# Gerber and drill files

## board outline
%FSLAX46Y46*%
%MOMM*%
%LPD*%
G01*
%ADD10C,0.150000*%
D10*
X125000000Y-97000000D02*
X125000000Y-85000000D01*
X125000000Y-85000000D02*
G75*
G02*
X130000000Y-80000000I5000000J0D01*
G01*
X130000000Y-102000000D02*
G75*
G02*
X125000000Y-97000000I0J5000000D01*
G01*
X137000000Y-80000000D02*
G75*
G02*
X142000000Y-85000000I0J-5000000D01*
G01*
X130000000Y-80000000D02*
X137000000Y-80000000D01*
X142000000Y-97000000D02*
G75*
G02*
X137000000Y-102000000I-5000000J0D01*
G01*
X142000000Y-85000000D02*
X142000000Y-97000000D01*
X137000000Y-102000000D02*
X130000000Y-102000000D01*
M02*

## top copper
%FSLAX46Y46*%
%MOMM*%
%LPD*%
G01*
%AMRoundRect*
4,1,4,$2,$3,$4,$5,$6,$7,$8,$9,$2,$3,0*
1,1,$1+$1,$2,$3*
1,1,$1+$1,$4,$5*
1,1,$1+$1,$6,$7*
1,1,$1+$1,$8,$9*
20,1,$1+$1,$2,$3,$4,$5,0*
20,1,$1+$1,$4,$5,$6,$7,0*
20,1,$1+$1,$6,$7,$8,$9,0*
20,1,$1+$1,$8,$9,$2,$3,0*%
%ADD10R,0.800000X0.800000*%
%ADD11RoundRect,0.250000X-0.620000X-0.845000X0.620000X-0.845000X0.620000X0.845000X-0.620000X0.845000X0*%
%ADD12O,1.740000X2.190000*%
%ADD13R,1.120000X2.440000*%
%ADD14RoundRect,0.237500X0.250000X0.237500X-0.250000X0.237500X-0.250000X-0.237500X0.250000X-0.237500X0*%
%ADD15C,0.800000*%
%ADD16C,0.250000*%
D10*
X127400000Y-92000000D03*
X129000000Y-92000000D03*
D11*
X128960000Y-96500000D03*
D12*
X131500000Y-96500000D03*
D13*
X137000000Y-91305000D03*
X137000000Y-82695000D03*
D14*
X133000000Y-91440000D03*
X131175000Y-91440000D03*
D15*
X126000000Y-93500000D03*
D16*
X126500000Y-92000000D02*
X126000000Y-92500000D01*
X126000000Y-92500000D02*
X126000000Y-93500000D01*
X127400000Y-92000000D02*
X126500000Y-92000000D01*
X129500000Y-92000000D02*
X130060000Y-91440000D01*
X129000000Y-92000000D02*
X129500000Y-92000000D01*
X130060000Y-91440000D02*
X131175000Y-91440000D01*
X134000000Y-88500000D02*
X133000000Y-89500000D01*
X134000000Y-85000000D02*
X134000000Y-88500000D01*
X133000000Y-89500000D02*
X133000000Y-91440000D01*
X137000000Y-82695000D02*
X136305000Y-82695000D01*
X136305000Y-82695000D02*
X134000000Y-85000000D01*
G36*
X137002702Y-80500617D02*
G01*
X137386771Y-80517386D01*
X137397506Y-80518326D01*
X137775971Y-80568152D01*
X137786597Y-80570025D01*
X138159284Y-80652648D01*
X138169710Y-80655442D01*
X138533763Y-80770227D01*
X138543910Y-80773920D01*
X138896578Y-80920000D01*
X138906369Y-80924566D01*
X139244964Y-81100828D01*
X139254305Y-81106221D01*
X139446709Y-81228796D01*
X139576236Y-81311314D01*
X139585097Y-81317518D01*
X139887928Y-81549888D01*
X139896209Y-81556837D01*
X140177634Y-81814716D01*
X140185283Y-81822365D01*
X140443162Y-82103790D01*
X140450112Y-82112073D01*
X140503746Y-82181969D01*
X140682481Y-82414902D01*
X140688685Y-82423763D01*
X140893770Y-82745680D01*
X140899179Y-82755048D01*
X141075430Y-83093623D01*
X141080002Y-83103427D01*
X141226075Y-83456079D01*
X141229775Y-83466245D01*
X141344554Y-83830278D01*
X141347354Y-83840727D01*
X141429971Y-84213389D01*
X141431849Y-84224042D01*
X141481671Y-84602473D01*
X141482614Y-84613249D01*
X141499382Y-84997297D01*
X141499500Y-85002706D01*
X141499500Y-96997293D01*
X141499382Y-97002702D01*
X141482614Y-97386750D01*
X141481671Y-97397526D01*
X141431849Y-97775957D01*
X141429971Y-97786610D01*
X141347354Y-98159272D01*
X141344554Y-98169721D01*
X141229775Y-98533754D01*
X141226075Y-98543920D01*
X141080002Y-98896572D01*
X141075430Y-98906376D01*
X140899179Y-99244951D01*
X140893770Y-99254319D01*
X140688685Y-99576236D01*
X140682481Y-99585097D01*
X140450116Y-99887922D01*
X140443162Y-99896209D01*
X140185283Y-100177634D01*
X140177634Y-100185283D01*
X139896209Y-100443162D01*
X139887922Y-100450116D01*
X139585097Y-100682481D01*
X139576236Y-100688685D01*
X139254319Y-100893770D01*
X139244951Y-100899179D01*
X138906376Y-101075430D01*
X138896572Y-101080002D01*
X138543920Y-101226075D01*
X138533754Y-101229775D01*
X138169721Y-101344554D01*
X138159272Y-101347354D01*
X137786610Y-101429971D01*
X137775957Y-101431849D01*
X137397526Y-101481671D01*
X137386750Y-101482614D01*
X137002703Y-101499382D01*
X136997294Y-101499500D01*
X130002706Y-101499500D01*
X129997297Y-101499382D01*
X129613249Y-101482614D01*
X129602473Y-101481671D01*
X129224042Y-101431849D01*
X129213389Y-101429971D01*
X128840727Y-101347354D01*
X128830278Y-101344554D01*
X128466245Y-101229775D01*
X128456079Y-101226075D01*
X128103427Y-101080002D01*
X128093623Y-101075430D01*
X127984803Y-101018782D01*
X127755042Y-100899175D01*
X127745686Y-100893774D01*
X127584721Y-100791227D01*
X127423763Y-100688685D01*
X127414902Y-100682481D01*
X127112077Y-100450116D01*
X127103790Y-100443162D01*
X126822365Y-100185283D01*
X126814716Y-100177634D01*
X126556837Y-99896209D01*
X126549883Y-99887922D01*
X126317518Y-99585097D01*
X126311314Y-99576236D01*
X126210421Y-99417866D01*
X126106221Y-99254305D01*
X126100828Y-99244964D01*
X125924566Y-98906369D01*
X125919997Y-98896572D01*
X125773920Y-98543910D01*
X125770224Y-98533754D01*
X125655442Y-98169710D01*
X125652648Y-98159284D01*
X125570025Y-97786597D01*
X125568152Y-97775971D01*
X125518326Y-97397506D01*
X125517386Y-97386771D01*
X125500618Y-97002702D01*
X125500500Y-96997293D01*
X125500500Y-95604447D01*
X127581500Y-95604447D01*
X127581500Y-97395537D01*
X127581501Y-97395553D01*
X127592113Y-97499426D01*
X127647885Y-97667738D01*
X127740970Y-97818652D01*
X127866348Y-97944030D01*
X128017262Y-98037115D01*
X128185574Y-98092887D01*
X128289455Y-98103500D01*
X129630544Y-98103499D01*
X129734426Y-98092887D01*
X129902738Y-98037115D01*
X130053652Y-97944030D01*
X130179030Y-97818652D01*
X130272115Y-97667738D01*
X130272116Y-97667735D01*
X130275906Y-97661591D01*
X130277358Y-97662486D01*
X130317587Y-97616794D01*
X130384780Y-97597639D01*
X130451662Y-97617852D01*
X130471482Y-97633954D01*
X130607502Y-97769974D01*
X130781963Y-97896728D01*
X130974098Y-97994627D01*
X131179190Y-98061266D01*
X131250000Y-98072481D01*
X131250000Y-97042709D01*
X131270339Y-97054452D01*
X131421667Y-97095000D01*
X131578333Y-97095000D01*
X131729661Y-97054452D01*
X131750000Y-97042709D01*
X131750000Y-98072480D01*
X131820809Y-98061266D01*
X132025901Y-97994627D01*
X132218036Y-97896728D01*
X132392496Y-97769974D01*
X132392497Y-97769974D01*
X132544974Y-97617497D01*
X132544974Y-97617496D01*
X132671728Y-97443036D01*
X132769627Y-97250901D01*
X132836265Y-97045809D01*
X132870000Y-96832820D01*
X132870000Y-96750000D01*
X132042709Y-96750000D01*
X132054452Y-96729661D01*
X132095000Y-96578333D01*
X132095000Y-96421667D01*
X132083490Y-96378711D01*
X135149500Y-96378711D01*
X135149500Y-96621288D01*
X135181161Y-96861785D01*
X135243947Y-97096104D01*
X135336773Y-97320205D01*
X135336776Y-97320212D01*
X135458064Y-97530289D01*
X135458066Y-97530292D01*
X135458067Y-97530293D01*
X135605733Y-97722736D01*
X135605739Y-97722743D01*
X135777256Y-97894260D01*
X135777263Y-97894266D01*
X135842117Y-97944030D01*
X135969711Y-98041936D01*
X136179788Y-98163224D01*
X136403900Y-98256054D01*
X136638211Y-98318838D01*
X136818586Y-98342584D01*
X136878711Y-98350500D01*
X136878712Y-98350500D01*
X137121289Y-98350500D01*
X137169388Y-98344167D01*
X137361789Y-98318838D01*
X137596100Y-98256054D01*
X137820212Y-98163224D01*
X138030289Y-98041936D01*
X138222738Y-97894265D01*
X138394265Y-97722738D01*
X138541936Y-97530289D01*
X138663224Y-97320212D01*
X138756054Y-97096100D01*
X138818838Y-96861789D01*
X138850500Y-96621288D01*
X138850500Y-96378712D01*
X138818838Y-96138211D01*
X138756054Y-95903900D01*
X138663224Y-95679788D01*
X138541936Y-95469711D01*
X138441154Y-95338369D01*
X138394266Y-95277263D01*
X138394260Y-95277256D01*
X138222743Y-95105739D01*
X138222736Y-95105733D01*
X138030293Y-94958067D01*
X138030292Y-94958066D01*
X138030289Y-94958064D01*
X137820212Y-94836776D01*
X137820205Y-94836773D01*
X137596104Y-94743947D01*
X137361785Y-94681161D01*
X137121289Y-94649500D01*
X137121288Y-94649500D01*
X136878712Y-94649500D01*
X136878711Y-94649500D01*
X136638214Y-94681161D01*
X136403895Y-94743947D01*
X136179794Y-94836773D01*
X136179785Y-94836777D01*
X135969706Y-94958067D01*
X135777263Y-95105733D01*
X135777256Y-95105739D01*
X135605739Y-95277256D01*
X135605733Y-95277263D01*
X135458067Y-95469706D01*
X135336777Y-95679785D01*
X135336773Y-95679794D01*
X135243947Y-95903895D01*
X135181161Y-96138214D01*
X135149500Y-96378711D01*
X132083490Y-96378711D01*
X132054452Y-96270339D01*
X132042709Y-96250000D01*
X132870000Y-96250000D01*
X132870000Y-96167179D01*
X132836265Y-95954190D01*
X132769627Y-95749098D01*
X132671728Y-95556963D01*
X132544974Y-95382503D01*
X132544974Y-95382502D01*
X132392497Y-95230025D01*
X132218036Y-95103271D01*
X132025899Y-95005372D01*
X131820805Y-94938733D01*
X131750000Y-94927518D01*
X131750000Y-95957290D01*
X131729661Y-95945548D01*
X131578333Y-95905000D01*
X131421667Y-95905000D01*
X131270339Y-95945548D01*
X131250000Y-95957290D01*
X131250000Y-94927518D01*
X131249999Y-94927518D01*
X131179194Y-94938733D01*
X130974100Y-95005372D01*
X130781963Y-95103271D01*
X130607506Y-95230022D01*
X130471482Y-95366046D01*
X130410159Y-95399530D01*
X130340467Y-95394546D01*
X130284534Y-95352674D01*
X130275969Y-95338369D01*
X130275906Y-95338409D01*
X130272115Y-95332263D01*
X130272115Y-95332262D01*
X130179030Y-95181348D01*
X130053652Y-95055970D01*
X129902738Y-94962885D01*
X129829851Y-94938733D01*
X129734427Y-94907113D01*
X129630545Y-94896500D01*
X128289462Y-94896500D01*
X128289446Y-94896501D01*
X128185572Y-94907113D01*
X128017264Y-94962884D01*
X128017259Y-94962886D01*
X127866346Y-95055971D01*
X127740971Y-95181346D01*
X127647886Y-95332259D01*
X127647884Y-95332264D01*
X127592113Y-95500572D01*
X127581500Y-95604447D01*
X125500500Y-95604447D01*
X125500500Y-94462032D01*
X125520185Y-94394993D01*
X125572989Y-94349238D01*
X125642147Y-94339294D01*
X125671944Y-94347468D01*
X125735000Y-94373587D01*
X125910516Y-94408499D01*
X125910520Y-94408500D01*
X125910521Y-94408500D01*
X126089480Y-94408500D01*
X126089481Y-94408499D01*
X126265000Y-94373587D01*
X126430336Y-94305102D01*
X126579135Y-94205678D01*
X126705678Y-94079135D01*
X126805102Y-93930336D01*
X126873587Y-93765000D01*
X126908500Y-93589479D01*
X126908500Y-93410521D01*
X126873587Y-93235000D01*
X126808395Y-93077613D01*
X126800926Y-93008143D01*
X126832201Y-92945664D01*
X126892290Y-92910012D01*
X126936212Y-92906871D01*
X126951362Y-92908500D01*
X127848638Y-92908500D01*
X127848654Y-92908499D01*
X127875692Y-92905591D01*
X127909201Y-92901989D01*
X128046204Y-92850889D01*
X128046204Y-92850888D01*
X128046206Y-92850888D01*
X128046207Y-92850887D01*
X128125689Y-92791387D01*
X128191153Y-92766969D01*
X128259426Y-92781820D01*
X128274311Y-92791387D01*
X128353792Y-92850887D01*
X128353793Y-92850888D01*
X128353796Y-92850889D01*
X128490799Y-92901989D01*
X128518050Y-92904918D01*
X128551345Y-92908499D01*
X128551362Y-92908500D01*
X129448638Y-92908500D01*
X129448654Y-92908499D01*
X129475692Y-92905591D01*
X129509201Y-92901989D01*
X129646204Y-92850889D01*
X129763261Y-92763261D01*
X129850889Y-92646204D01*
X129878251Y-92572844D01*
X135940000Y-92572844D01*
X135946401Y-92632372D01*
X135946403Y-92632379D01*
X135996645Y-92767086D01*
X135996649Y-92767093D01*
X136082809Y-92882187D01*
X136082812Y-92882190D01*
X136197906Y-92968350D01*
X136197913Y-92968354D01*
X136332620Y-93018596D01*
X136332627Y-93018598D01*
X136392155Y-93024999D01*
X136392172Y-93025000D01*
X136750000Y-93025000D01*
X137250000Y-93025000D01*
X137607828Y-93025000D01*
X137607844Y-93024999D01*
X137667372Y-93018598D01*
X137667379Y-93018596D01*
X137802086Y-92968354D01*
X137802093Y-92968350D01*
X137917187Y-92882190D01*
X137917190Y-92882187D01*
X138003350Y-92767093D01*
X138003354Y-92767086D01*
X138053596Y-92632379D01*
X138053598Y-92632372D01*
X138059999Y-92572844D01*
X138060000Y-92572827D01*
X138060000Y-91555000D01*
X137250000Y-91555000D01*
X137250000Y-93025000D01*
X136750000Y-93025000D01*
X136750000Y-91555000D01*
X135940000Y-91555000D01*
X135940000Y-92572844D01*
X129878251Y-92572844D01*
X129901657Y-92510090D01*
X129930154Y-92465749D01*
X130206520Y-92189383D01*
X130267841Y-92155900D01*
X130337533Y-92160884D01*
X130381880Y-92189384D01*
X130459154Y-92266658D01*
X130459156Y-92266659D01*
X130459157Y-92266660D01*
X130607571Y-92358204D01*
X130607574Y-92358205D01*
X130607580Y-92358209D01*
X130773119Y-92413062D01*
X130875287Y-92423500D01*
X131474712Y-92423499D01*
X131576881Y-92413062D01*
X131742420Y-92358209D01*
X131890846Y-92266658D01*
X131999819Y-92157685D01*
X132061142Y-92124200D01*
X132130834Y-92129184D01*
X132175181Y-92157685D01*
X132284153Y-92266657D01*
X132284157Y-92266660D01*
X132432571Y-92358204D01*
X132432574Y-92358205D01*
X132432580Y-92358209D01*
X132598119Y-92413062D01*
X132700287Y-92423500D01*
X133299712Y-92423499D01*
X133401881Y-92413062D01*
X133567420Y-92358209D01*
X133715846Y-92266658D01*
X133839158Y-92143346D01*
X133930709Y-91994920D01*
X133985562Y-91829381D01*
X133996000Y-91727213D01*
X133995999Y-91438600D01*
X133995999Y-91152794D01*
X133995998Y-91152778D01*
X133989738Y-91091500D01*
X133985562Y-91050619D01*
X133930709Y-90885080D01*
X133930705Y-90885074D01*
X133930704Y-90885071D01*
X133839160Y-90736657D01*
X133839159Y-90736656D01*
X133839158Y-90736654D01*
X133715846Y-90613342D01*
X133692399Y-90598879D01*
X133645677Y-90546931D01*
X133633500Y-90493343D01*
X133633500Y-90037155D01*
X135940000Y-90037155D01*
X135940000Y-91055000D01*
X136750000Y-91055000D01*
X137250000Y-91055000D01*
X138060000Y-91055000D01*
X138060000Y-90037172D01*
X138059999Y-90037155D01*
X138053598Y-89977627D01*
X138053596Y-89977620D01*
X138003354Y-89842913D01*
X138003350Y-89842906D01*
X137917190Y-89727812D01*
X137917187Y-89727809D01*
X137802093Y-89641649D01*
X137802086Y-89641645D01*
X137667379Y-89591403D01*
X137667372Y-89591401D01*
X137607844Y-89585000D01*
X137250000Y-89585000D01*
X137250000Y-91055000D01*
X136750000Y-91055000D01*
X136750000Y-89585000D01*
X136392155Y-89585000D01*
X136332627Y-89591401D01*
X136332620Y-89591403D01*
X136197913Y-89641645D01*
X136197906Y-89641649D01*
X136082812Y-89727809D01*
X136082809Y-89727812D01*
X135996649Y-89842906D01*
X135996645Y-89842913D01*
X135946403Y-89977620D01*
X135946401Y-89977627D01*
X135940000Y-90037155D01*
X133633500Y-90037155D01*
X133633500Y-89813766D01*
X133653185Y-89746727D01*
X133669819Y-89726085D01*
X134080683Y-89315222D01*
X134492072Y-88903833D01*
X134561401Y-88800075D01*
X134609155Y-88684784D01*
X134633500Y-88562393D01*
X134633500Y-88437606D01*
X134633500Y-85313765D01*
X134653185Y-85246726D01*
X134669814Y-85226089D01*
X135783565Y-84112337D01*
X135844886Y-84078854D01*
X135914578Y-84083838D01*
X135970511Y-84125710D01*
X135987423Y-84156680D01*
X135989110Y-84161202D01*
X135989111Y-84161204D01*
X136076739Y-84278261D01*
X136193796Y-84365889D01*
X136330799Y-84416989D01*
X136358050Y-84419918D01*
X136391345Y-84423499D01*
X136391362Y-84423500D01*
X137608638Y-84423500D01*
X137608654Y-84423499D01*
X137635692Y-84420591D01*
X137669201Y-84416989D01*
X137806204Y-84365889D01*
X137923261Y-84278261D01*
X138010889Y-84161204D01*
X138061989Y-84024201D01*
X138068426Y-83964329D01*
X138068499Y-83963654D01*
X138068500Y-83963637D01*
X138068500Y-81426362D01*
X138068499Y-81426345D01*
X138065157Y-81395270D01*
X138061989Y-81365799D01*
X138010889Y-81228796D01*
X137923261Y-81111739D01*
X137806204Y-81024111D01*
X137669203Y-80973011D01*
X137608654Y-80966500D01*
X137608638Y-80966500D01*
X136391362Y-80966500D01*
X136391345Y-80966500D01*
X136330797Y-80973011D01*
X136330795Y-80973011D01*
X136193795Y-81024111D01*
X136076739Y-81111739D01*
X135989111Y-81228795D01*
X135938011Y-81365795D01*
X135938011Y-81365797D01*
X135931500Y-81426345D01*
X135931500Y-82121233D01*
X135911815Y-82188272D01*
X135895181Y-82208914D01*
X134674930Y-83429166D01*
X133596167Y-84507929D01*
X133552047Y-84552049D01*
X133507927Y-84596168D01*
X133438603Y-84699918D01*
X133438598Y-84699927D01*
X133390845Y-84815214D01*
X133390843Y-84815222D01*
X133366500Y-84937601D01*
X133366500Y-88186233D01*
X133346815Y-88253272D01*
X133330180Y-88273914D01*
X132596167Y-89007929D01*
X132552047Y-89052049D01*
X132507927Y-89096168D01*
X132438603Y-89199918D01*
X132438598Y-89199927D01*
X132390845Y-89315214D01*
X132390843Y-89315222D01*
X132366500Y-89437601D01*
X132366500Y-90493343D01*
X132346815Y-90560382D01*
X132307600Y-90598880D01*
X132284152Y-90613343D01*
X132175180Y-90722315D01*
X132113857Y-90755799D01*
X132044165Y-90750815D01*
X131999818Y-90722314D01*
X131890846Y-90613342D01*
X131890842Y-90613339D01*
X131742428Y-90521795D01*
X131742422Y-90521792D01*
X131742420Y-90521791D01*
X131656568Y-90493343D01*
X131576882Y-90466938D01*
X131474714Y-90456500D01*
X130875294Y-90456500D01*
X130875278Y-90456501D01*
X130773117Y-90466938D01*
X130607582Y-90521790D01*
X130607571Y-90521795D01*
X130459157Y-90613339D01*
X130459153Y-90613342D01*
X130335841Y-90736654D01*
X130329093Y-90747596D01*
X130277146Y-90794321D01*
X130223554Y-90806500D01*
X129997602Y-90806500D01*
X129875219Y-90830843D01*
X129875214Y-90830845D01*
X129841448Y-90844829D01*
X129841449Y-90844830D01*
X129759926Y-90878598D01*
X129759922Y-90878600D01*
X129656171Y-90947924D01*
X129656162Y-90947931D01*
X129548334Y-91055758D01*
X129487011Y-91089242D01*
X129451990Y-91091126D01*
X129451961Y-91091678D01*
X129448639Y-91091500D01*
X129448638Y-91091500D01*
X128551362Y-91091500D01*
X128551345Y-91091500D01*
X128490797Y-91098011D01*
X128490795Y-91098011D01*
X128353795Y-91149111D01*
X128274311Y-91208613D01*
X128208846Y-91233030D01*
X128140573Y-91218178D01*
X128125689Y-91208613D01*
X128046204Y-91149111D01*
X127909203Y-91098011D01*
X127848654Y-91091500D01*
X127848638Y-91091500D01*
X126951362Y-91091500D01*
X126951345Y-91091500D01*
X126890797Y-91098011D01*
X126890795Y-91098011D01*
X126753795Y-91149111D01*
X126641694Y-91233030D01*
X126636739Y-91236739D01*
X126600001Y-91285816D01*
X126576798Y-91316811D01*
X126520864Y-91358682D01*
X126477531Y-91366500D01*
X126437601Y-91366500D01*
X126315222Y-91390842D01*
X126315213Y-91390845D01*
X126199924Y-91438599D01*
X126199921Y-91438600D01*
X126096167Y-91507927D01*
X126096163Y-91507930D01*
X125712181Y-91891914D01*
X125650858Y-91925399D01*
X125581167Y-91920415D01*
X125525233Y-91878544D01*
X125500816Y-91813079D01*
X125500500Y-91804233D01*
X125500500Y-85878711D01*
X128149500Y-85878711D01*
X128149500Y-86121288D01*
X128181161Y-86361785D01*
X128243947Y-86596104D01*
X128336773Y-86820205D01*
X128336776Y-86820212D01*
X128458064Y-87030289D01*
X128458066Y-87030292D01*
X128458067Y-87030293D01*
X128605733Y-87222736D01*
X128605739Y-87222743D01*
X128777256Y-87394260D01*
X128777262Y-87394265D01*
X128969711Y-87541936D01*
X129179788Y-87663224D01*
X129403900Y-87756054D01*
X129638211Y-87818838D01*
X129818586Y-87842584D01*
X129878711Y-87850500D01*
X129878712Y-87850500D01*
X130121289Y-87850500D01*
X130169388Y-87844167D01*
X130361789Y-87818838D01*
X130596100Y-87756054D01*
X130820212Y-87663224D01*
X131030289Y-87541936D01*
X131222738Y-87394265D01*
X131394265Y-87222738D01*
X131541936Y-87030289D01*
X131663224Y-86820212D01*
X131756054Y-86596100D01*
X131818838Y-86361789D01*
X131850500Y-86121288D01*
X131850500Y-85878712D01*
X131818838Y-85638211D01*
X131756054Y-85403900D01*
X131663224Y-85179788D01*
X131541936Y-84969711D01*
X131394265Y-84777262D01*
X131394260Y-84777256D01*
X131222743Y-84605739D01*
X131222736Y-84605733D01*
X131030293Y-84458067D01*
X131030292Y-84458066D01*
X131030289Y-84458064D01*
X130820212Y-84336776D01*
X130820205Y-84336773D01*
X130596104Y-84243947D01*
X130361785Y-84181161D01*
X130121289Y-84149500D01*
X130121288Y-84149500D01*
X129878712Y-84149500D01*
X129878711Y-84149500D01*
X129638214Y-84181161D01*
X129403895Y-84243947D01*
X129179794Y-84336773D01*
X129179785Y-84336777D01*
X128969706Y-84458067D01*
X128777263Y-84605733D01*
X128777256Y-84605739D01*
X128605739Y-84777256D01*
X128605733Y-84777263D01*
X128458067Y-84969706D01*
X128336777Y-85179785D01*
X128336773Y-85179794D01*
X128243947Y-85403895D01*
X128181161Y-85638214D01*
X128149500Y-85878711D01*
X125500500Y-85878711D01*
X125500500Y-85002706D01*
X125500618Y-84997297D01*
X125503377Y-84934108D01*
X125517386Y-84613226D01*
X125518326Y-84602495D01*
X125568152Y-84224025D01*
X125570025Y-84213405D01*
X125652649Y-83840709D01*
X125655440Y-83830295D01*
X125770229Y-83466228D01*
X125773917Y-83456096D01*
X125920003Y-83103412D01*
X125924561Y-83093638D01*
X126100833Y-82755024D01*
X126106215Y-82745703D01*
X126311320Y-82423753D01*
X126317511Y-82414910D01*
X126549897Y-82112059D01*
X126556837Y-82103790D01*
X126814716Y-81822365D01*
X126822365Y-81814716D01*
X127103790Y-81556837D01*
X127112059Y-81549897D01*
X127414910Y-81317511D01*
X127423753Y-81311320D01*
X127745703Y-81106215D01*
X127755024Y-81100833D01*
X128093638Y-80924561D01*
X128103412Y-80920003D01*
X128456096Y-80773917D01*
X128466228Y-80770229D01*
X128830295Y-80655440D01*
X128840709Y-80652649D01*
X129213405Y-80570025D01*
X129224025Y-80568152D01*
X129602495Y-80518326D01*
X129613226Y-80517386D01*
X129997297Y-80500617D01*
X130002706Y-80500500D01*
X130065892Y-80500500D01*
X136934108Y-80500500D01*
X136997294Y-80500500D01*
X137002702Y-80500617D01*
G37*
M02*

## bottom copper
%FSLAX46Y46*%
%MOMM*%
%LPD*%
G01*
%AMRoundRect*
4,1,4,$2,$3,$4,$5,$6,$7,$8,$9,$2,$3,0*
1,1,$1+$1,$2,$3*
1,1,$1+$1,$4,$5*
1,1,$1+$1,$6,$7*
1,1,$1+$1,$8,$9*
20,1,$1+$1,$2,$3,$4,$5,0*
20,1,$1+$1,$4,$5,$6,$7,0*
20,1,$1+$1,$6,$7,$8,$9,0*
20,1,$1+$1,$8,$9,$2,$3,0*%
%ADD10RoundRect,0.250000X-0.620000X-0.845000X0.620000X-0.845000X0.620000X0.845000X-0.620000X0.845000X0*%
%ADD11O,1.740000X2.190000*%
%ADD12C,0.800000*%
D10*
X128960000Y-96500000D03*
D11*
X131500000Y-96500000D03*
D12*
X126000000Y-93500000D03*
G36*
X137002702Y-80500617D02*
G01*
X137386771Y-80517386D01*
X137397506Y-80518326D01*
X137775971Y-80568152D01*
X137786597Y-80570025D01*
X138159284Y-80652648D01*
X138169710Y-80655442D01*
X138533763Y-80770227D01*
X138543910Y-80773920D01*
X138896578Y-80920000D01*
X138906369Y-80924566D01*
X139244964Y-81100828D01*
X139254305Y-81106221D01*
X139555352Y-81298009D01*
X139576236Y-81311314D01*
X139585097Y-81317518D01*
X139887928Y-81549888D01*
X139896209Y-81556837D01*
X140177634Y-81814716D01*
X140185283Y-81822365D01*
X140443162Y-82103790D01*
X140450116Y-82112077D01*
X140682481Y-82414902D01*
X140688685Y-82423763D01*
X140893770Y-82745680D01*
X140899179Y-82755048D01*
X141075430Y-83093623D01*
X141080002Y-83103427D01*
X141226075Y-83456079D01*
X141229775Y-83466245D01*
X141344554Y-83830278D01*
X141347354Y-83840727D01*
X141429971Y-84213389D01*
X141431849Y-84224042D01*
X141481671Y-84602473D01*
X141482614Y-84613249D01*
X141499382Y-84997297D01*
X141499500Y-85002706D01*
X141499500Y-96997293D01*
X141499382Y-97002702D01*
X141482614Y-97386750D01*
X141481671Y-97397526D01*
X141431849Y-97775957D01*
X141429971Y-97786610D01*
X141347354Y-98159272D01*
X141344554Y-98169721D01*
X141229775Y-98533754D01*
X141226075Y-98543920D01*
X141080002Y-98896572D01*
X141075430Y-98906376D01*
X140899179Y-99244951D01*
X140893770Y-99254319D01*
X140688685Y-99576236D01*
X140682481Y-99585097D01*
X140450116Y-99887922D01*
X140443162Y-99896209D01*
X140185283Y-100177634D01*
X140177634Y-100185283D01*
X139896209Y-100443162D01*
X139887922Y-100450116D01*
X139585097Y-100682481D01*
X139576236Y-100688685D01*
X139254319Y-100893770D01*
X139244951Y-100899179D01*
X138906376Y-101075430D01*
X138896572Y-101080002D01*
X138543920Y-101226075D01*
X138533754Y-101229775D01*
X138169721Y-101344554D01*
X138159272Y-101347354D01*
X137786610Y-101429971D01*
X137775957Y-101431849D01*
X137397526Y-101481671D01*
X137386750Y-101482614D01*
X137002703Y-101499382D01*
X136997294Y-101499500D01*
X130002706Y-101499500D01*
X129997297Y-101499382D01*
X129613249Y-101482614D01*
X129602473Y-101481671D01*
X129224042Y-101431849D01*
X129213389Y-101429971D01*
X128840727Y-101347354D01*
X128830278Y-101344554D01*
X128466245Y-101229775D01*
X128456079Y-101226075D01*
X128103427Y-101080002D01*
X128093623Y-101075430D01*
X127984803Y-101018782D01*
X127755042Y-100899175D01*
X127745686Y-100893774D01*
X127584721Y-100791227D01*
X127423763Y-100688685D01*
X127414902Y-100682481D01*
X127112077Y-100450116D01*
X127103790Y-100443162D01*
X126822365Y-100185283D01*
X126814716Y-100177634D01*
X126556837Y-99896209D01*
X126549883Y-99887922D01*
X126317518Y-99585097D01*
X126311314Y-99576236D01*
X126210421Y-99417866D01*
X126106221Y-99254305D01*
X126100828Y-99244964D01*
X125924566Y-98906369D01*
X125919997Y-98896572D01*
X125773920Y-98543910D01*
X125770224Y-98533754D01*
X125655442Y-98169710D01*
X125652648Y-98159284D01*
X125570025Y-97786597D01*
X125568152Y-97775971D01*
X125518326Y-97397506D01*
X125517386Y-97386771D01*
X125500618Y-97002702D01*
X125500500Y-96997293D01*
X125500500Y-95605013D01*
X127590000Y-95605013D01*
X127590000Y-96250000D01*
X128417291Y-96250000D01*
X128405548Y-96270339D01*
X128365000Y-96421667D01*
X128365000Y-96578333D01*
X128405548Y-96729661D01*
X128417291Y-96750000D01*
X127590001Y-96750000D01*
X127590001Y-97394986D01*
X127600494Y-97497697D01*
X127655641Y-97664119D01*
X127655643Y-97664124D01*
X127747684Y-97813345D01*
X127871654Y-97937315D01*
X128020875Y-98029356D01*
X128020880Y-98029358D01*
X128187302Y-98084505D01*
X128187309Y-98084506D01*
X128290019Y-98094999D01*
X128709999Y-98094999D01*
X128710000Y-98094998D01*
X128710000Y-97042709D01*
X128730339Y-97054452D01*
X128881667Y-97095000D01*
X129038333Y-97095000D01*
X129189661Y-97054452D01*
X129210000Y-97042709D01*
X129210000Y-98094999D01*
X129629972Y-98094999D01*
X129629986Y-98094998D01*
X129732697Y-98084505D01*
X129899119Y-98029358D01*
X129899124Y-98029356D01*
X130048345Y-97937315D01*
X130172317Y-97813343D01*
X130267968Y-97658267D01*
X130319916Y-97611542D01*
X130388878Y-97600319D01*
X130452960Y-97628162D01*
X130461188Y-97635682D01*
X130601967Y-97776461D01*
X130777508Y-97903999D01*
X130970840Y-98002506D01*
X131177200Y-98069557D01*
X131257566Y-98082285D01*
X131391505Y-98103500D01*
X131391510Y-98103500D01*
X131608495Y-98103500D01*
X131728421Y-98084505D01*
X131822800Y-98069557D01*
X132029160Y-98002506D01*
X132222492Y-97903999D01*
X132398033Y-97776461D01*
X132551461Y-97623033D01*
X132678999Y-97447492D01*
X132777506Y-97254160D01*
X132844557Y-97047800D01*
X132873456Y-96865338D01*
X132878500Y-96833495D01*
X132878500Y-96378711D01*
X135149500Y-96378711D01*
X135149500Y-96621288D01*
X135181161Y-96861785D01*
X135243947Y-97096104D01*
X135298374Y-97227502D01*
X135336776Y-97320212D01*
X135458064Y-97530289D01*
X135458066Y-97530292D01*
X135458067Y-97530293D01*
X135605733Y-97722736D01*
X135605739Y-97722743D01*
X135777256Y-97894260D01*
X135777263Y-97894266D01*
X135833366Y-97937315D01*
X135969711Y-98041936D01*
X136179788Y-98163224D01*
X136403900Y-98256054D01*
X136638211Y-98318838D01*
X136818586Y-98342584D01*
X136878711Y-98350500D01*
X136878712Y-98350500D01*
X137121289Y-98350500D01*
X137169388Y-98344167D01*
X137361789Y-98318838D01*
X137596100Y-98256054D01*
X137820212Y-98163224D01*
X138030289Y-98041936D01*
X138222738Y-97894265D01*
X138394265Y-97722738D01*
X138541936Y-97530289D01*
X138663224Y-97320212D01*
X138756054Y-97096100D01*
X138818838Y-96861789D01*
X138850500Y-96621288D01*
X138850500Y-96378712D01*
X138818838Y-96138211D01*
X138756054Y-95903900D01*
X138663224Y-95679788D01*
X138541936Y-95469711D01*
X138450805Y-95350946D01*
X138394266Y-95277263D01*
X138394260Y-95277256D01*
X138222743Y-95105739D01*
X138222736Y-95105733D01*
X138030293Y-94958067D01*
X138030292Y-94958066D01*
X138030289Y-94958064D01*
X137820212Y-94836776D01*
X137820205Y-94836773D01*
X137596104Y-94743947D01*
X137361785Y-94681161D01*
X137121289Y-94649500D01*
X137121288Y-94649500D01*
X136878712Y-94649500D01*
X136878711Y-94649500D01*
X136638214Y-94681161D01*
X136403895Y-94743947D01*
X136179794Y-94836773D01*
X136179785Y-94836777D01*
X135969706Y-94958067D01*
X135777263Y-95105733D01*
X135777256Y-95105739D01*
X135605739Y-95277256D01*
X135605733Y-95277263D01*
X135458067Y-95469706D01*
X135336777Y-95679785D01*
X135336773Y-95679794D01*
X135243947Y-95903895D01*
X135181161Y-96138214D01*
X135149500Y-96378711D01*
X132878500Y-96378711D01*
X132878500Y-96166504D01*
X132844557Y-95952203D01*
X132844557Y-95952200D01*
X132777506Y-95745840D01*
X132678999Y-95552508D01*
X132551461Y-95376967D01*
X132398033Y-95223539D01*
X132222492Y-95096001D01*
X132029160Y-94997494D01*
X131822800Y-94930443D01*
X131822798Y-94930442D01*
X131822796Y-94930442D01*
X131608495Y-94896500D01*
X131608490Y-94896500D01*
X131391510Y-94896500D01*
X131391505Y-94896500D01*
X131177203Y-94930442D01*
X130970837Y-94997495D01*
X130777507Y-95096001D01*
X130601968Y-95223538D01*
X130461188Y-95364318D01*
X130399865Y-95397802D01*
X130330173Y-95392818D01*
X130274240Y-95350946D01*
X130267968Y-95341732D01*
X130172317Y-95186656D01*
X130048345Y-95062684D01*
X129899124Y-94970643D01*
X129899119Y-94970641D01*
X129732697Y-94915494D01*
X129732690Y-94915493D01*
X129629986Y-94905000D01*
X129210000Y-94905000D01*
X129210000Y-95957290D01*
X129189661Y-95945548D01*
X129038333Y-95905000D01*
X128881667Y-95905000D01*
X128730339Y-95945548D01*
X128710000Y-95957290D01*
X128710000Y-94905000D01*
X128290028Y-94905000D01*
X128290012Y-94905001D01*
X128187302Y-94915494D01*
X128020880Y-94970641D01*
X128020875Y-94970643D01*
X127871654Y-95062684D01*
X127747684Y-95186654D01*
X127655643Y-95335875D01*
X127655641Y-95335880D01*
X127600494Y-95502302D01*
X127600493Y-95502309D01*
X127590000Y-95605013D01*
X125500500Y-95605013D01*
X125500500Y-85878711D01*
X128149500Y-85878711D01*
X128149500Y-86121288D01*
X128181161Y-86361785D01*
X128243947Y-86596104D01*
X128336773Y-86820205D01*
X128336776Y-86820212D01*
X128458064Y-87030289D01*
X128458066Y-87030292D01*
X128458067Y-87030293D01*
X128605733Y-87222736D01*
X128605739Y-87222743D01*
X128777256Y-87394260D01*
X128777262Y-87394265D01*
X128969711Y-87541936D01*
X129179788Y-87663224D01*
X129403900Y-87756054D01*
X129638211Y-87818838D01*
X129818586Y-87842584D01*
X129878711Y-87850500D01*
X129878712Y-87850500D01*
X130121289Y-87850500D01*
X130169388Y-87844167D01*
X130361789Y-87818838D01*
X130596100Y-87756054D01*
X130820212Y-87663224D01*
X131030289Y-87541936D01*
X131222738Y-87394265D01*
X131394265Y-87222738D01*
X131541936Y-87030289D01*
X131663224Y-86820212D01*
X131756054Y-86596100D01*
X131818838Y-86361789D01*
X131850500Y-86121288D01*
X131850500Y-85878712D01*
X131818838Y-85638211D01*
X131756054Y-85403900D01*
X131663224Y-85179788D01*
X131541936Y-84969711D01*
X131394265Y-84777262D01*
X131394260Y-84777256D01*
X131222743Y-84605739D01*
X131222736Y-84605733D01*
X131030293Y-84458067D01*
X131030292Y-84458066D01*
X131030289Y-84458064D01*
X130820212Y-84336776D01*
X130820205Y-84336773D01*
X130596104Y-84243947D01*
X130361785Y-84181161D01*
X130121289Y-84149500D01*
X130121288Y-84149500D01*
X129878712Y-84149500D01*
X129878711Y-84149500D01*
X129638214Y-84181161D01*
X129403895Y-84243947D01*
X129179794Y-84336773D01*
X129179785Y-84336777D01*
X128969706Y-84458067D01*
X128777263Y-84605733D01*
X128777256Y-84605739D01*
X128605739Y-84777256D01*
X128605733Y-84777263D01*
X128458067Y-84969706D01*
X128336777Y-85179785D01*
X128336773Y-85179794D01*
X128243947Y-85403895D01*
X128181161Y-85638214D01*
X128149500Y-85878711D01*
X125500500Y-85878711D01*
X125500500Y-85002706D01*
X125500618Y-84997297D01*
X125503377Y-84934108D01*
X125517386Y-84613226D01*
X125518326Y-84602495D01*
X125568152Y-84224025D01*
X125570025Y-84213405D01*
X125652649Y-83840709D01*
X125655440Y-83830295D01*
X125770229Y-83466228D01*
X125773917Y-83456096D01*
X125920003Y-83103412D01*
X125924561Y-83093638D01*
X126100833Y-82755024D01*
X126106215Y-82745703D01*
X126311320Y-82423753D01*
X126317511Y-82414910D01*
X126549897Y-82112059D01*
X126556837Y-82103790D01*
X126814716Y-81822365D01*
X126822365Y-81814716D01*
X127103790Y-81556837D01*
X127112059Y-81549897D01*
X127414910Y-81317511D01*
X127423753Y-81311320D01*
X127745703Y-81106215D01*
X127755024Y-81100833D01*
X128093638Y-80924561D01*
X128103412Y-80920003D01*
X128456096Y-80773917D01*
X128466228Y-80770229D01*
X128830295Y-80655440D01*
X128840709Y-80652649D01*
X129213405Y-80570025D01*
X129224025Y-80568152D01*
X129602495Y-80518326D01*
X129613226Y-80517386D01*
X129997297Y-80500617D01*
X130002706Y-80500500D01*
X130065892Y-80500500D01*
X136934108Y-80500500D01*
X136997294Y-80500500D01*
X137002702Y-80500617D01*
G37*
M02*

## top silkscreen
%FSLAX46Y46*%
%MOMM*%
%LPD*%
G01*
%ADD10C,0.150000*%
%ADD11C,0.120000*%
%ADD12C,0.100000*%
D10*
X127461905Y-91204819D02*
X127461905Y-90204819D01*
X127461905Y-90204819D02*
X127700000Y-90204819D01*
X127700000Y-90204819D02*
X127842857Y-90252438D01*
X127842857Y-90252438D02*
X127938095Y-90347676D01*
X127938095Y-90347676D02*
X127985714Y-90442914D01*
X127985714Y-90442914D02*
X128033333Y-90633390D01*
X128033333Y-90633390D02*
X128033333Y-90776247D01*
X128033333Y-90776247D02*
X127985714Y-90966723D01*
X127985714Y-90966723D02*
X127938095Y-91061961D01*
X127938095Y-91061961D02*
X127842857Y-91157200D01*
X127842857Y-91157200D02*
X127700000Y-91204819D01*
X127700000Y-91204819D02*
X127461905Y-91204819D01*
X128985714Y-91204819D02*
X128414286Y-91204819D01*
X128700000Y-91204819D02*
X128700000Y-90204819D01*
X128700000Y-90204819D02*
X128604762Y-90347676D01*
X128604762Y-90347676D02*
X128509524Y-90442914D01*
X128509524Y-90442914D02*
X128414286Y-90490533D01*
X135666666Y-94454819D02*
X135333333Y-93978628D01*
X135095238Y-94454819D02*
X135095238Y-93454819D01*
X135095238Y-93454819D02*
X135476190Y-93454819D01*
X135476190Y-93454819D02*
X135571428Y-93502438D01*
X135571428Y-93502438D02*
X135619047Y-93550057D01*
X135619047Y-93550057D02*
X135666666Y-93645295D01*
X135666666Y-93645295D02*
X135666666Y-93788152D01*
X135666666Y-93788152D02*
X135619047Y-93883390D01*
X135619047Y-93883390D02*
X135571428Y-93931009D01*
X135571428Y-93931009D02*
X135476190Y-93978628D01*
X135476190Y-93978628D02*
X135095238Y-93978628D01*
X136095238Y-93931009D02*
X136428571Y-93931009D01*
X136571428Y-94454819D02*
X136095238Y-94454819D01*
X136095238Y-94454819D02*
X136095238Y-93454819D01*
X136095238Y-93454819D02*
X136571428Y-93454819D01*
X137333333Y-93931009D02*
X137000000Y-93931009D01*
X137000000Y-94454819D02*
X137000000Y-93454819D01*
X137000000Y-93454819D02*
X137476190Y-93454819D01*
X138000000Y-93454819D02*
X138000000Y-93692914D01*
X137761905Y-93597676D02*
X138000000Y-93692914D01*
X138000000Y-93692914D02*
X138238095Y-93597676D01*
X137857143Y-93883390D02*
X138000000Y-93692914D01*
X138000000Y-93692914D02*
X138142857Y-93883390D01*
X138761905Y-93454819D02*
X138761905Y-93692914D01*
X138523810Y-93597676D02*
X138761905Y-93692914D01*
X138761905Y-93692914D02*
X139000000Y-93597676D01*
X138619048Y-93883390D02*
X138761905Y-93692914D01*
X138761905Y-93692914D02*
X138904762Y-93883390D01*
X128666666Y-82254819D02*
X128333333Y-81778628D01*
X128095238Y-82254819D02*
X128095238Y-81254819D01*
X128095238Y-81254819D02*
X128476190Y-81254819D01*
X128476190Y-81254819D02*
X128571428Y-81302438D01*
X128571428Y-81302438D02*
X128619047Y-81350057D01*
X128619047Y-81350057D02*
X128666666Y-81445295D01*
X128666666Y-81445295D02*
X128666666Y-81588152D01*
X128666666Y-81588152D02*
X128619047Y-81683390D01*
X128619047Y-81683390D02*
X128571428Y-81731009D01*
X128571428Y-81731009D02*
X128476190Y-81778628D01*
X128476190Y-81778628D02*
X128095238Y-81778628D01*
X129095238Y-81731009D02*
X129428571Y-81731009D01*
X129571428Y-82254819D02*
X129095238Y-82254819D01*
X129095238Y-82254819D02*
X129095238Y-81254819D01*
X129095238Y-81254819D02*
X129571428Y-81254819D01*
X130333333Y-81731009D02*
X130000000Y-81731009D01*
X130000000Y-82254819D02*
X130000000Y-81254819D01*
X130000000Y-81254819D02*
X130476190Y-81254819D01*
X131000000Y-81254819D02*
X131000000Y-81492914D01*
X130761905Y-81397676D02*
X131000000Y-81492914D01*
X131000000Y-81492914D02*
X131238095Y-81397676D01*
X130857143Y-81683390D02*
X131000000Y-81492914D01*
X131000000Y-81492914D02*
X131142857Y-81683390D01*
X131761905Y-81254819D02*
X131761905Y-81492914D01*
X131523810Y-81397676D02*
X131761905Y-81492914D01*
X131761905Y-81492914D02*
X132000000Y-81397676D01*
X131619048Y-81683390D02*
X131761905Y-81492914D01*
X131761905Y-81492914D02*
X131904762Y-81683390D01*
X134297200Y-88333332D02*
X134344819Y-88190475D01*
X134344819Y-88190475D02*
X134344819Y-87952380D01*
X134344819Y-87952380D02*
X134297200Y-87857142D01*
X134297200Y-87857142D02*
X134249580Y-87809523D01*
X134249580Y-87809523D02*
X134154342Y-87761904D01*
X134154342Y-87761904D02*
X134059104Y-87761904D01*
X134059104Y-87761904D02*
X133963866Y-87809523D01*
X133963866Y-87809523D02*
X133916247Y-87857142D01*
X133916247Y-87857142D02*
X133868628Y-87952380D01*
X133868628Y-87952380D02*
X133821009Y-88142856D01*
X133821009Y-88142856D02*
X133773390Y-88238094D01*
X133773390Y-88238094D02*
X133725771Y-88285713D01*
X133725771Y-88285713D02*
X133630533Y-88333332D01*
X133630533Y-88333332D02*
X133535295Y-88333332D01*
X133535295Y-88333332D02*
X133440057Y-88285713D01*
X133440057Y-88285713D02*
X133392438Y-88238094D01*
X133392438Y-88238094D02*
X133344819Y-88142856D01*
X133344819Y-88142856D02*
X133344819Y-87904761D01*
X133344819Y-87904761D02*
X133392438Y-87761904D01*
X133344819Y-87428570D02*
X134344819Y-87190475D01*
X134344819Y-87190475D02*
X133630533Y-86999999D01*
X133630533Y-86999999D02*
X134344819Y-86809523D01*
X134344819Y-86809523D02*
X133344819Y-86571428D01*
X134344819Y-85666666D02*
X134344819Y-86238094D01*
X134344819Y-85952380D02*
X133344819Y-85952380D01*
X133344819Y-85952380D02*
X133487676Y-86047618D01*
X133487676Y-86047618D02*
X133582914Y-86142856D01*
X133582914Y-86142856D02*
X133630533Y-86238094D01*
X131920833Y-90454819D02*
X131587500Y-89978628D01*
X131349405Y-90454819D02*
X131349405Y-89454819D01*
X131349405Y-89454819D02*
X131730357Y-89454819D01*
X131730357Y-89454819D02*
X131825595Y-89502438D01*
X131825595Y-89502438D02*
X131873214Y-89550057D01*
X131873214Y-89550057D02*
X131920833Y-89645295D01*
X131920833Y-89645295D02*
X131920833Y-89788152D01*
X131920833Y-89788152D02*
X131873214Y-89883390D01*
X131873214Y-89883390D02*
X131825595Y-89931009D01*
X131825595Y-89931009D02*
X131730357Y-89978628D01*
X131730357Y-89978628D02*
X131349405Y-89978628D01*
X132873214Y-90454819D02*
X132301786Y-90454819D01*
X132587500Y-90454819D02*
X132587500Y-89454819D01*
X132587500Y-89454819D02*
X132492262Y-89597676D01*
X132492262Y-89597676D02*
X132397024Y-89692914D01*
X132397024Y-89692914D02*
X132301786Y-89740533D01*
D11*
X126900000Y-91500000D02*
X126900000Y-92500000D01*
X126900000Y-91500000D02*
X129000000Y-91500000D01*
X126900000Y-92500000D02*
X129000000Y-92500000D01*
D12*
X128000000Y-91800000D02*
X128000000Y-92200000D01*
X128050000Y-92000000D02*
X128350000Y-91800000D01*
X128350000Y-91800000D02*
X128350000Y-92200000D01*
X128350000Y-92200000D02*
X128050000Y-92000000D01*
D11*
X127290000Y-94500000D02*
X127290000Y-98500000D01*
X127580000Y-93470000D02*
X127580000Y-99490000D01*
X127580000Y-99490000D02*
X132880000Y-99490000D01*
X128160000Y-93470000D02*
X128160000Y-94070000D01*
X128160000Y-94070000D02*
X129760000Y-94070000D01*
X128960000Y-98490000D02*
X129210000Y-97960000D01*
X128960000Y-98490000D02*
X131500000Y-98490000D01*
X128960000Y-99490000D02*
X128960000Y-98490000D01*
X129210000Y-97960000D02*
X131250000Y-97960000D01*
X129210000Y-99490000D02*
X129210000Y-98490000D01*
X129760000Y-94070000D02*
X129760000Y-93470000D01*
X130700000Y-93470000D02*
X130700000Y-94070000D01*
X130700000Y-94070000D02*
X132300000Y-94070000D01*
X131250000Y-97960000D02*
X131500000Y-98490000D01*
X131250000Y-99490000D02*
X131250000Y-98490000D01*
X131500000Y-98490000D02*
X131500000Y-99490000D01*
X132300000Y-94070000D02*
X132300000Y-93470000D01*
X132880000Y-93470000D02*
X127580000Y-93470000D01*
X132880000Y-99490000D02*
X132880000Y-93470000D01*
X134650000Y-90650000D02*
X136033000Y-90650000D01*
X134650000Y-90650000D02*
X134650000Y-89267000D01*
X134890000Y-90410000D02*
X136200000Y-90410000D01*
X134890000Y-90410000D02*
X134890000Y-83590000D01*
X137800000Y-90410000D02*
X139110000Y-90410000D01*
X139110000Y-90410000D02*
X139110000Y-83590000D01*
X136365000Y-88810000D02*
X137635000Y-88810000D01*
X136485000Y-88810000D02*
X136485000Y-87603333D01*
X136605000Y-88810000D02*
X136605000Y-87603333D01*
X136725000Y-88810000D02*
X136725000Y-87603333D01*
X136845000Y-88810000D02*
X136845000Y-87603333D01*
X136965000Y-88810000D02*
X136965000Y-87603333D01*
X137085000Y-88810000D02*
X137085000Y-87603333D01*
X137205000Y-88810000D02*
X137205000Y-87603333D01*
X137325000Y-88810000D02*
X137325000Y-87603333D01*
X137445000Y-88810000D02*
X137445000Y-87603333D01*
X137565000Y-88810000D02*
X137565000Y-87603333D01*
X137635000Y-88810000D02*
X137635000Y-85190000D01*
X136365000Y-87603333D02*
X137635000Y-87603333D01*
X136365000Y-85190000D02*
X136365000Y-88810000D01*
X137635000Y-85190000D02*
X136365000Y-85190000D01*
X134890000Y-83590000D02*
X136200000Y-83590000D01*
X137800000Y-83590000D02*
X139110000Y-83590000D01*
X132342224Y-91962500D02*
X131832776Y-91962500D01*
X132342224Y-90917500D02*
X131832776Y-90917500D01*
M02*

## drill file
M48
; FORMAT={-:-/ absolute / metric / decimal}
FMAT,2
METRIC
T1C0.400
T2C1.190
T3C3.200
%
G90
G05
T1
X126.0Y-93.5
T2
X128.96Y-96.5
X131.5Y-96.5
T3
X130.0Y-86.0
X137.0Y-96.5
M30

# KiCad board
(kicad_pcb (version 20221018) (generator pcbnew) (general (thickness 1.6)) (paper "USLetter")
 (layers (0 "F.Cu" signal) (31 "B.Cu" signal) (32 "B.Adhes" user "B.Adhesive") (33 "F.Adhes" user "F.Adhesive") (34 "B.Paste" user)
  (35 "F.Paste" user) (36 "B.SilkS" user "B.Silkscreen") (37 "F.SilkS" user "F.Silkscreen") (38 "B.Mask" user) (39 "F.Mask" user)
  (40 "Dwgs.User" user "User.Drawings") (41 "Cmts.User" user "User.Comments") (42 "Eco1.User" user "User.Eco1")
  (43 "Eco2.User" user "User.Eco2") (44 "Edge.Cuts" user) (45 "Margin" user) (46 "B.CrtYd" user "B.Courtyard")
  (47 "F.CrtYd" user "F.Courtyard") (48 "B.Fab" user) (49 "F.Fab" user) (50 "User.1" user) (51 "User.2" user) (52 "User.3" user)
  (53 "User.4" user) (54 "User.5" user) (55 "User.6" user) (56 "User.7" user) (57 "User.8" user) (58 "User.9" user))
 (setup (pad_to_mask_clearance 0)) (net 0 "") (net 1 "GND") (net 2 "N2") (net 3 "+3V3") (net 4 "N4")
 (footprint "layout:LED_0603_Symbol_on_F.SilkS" (layer "F.Cu") (at 128.2 92)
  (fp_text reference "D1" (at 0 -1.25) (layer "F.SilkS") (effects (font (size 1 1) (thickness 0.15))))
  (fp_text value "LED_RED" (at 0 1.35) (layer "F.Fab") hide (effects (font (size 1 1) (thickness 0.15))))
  (fp_line (start -1.3 -0.5) (end -1.3 0.5) (stroke (width 0.12) (type solid)) (layer "F.SilkS"))
  (fp_line (start -1.3 -0.5) (end 0.8 -0.5) (stroke (width 0.12) (type solid)) (layer "F.SilkS"))
  (fp_line (start -1.3 0.5) (end 0.8 0.5) (stroke (width 0.12) (type solid)) (layer "F.SilkS"))
  (fp_line (start -0.2 -0.2) (end -0.2 0.2) (stroke (width 0.1) (type solid)) (layer "F.SilkS"))
  (fp_line (start -0.15 0) (end 0.15 -0.2) (stroke (width 0.1) (type solid)) (layer "F.SilkS"))
  (fp_line (start 0.15 -0.2) (end 0.15 0.2) (stroke (width 0.1) (type solid)) (layer "F.SilkS"))
  (fp_line (start 0.15 0.2) (end -0.15 0) (stroke (width 0.1) (type solid)) (layer "F.SilkS"))
  (pad "1" smd rect (at -0.8 0 180) (size 0.8 0.8) (layers "F.Cu" "F.Paste" "F.Mask") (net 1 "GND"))
  (pad "2" smd rect (at 0.8 0 180) (size 0.8 0.8) (layers "F.Cu" "F.Paste" "F.Mask") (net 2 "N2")))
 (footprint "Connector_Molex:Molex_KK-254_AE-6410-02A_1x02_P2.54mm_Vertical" (layer "F.Cu") (at 128.96 96.5)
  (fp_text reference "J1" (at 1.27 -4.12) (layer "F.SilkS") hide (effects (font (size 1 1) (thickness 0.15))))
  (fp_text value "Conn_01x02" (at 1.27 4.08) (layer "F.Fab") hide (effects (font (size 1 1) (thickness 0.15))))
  (fp_line (start -1.67 -2) (end -1.67 2) (stroke (width 0.12) (type solid)) (layer "F.SilkS"))
  (fp_line (start -1.38 -3.03) (end -1.38 2.99) (stroke (width 0.12) (type solid)) (layer "F.SilkS"))
  (fp_line (start -1.38 2.99) (end 3.92 2.99) (stroke (width 0.12) (type solid)) (layer "F.SilkS"))
  (fp_line (start -0.8 -3.03) (end -0.8 -2.43) (stroke (width 0.12) (type solid)) (layer "F.SilkS"))
  (fp_line (start -0.8 -2.43) (end 0.8 -2.43) (stroke (width 0.12) (type solid)) (layer "F.SilkS"))
  (fp_line (start 0 1.99) (end 0.25 1.46) (stroke (width 0.12) (type solid)) (layer "F.SilkS"))
  (fp_line (start 0 1.99) (end 2.54 1.99) (stroke (width 0.12) (type solid)) (layer "F.SilkS"))
  (fp_line (start 0 2.99) (end 0 1.99) (stroke (width 0.12) (type solid)) (layer "F.SilkS"))
  (fp_line (start 0.25 1.46) (end 2.29 1.46) (stroke (width 0.12) (type solid)) (layer "F.SilkS"))
  (fp_line (start 0.25 2.99) (end 0.25 1.99) (stroke (width 0.12) (type solid)) (layer "F.SilkS"))
  (fp_line (start 0.8 -2.43) (end 0.8 -3.03) (stroke (width 0.12) (type solid)) (layer "F.SilkS"))
  (fp_line (start 1.74 -3.03) (end 1.74 -2.43) (stroke (width 0.12) (type solid)) (layer "F.SilkS"))
  (fp_line (start 1.74 -2.43) (end 3.34 -2.43) (stroke (width 0.12) (type solid)) (layer "F.SilkS"))
  (fp_line (start 2.29 1.46) (end 2.54 1.99) (stroke (width 0.12) (type solid)) (layer "F.SilkS"))
  (fp_line (start 2.29 2.99) (end 2.29 1.99) (stroke (width 0.12) (type solid)) (layer "F.SilkS"))
  (fp_line (start 2.54 1.99) (end 2.54 2.99) (stroke (width 0.12) (type solid)) (layer "F.SilkS"))
  (fp_line (start 3.34 -2.43) (end 3.34 -3.03) (stroke (width 0.12) (type solid)) (layer "F.SilkS"))
  (fp_line (start 3.92 -3.03) (end -1.38 -3.03) (stroke (width 0.12) (type solid)) (layer "F.SilkS"))
  (fp_line (start 3.92 2.99) (end 3.92 -3.03) (stroke (width 0.12) (type solid)) (layer "F.SilkS"))
  (pad "1" thru_hole roundrect (at 0 0) (size 1.74 2.19) (drill 1.19) (layers "*.Cu" "*.Mask") (roundrect_rratio 0.143678) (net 1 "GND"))
  (pad "2" thru_hole oval (at 2.54 0) (size 1.74 2.19) (drill 1.19) (layers "*.Cu" "*.Mask") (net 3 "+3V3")))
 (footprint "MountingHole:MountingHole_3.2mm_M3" (layer "F.Cu") (at 137 96.5)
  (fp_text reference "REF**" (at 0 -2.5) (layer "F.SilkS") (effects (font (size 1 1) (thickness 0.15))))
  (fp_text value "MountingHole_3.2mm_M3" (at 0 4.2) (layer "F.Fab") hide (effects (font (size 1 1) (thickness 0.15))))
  (pad "" np_thru_hole circle (at 0 0) (size 3.2 3.2) (drill 3.2) (layers "*.Cu" "*.Mask")))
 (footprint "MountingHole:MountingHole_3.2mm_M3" (layer "F.Cu") (at 130 86)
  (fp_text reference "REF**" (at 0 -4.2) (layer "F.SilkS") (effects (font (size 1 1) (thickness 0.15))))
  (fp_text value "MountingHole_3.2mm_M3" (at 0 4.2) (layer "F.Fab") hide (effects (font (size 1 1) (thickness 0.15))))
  (pad "" np_thru_hole circle (at 0 0) (size 3.2 3.2) (drill 3.2) (layers "*.Cu" "*.Mask")))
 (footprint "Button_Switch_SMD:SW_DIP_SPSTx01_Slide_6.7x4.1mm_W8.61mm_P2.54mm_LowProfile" (layer "F.Cu") (at 137 87 90)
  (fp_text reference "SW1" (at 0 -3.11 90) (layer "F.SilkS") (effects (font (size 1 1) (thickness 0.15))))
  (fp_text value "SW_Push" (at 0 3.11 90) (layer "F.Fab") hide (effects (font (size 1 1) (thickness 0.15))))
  (fp_line (start -3.65 -2.35) (end -3.65 -0.967) (stroke (width 0.12) (type solid)) (layer "F.SilkS"))
  (fp_line (start -3.65 -2.35) (end -2.267 -2.35) (stroke (width 0.12) (type solid)) (layer "F.SilkS"))
  (fp_line (start -3.41 -2.11) (end -3.41 -0.8) (stroke (width 0.12) (type solid)) (layer "F.SilkS"))
  (fp_line (start -3.41 -2.11) (end 3.41 -2.11) (stroke (width 0.12) (type solid)) (layer "F.SilkS"))
  (fp_line (start -3.41 0.8) (end -3.41 2.11) (stroke (width 0.12) (type solid)) (layer "F.SilkS"))
  (fp_line (start -3.41 2.11) (end 3.41 2.11) (stroke (width 0.12) (type solid)) (layer "F.SilkS"))
  (fp_line (start -1.81 -0.635) (end -1.81 0.635) (stroke (width 0.12) (type solid)) (layer "F.SilkS"))
  (fp_line (start -1.81 -0.515) (end -0.603333 -0.515) (stroke (width 0.12) (type solid)) (layer "F.SilkS"))
  (fp_line (start -1.81 -0.395) (end -0.603333 -0.395) (stroke (width 0.12) (type solid)) (layer "F.SilkS"))
  (fp_line (start -1.81 -0.275) (end -0.603333 -0.275) (stroke (width 0.12) (type solid)) (layer "F.SilkS"))
  (fp_line (start -1.81 -0.155) (end -0.603333 -0.155) (stroke (width 0.12) (type solid)) (layer "F.SilkS"))
  (fp_line (start -1.81 -0.035) (end -0.603333 -0.035) (stroke (width 0.12) (type solid)) (layer "F.SilkS"))
  (fp_line (start -1.81 0.085) (end -0.603333 0.085) (stroke (width 0.12) (type solid)) (layer "F.SilkS"))
  (fp_line (start -1.81 0.205) (end -0.603333 0.205) (stroke (width 0.12) (type solid)) (layer "F.SilkS"))
  (fp_line (start -1.81 0.325) (end -0.603333 0.325) (stroke (width 0.12) (type solid)) (layer "F.SilkS"))
  (fp_line (start -1.81 0.445) (end -0.603333 0.445) (stroke (width 0.12) (type solid)) (layer "F.SilkS"))
  (fp_line (start -1.81 0.565) (end -0.603333 0.565) (stroke (width 0.12) (type solid)) (layer "F.SilkS"))
  (fp_line (start -1.81 0.635) (end 1.81 0.635) (stroke (width 0.12) (type solid)) (layer "F.SilkS"))
  (fp_line (start -0.603333 -0.635) (end -0.603333 0.635) (stroke (width 0.12) (type solid)) (layer "F.SilkS"))
  (fp_line (start 1.81 -0.635) (end -1.81 -0.635) (stroke (width 0.12) (type solid)) (layer "F.SilkS"))
  (fp_line (start 1.81 0.635) (end 1.81 -0.635) (stroke (width 0.12) (type solid)) (layer "F.SilkS"))
  (fp_line (start 3.41 -2.11) (end 3.41 -0.8) (stroke (width 0.12) (type solid)) (layer "F.SilkS"))
  (fp_line (start 3.41 0.8) (end 3.41 2.11) (stroke (width 0.12) (type solid)) (layer "F.SilkS"))
  (pad "1" smd rect (at -4.305 0 90) (size 2.44 1.12) (layers "F.Cu" "F.Paste" "F.Mask") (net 3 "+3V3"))
  (pad "2" smd rect (at 4.305 0 90) (size 2.44 1.12) (layers "F.Cu" "F.Paste" "F.Mask") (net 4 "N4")))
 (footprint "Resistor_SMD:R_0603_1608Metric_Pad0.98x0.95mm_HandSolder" (layer "F.Cu") (at 132.0875 91.44 180)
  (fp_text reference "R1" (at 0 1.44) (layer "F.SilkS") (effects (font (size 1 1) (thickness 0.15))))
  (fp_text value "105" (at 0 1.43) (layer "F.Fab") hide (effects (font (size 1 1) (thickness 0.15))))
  (fp_line (start -0.254724 -0.5225) (end 0.254724 -0.5225) (stroke (width 0.12) (type solid)) (layer "F.SilkS"))
  (fp_line (start -0.254724 0.5225) (end 0.254724 0.5225) (stroke (width 0.12) (type solid)) (layer "F.SilkS"))
  (pad "1" smd roundrect (at -0.9125 0 180) (size 0.975 0.95) (layers "F.Cu" "F.Paste" "F.Mask") (roundrect_rratio 0.25) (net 4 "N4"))
  (pad "2" smd roundrect (at 0.9125 0 180) (size 0.975 0.95) (layers "F.Cu" "F.Paste" "F.Mask") (roundrect_rratio 0.25) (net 2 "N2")))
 (gr_line (start 125 97) (end 125 85) (stroke (width 0.15) (type default)) (layer "Edge.Cuts"))
 (gr_arc (start 125 85) (mid 126.464466 81.464467) (end 130 80) (stroke (width 0.15) (type default)) (layer "Edge.Cuts"))
 (gr_arc (start 130 102) (mid 126.464467 100.535534) (end 125 97) (stroke (width 0.15) (type default)) (layer "Edge.Cuts"))
 (gr_arc (start 137 80) (mid 140.535533 81.464466) (end 142 85) (stroke (width 0.15) (type default)) (layer "Edge.Cuts"))
 (gr_line (start 130 80) (end 137 80) (stroke (width 0.15) (type default)) (layer "Edge.Cuts"))
 (gr_arc (start 142 97) (mid 140.535534 100.535533) (end 137 102) (stroke (width 0.15) (type default)) (layer "Edge.Cuts"))
 (gr_line (start 142 85) (end 142 97) (stroke (width 0.15) (type default)) (layer "Edge.Cuts"))
 (gr_line (start 137 102) (end 130 102) (stroke (width 0.15) (type default)) (layer "Edge.Cuts"))
 (segment (start 126.5 92) (end 126 92.5) (width 0.25) (layer "F.Cu") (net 1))
 (segment (start 126 92.5) (end 126 93.5) (width 0.25) (layer "F.Cu") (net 1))
 (segment (start 127.4 92) (end 126.5 92) (width 0.25) (layer "F.Cu") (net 1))
 (via (at 126 93.5) (size 0.8) (drill 0.4) (layers "F.Cu" "B.Cu") (free) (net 1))
 (segment (start 129.5 92) (end 130.06 91.44) (width 0.25) (layer "F.Cu") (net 2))
 (segment (start 129 92) (end 129.5 92) (width 0.25) (layer "F.Cu") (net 2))
 (segment (start 130.06 91.44) (end 131.175 91.44) (width 0.25) (layer "F.Cu") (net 2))
 (segment (start 134 88.5) (end 133 89.5) (width 0.25) (layer "F.Cu") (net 4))
 (segment (start 134 85) (end 134 88.5) (width 0.25) (layer "F.Cu") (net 4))
 (segment (start 133 89.5) (end 133 91.44) (width 0.25) (layer "F.Cu") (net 4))
 (segment (start 137 82.695) (end 136.305 82.695) (width 0.25) (layer "F.Cu") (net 4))
 (segment (start 136.305 82.695) (end 134 85) (width 0.25) (layer "F.Cu") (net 4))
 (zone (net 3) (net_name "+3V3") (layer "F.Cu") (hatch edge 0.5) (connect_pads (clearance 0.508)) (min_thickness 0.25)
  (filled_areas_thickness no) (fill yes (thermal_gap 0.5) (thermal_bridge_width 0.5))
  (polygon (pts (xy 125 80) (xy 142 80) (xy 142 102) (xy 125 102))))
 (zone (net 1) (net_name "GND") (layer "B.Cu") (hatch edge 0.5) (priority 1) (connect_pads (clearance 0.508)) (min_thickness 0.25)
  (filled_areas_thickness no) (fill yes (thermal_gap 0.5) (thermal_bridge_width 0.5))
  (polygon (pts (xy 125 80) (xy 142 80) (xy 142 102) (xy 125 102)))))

